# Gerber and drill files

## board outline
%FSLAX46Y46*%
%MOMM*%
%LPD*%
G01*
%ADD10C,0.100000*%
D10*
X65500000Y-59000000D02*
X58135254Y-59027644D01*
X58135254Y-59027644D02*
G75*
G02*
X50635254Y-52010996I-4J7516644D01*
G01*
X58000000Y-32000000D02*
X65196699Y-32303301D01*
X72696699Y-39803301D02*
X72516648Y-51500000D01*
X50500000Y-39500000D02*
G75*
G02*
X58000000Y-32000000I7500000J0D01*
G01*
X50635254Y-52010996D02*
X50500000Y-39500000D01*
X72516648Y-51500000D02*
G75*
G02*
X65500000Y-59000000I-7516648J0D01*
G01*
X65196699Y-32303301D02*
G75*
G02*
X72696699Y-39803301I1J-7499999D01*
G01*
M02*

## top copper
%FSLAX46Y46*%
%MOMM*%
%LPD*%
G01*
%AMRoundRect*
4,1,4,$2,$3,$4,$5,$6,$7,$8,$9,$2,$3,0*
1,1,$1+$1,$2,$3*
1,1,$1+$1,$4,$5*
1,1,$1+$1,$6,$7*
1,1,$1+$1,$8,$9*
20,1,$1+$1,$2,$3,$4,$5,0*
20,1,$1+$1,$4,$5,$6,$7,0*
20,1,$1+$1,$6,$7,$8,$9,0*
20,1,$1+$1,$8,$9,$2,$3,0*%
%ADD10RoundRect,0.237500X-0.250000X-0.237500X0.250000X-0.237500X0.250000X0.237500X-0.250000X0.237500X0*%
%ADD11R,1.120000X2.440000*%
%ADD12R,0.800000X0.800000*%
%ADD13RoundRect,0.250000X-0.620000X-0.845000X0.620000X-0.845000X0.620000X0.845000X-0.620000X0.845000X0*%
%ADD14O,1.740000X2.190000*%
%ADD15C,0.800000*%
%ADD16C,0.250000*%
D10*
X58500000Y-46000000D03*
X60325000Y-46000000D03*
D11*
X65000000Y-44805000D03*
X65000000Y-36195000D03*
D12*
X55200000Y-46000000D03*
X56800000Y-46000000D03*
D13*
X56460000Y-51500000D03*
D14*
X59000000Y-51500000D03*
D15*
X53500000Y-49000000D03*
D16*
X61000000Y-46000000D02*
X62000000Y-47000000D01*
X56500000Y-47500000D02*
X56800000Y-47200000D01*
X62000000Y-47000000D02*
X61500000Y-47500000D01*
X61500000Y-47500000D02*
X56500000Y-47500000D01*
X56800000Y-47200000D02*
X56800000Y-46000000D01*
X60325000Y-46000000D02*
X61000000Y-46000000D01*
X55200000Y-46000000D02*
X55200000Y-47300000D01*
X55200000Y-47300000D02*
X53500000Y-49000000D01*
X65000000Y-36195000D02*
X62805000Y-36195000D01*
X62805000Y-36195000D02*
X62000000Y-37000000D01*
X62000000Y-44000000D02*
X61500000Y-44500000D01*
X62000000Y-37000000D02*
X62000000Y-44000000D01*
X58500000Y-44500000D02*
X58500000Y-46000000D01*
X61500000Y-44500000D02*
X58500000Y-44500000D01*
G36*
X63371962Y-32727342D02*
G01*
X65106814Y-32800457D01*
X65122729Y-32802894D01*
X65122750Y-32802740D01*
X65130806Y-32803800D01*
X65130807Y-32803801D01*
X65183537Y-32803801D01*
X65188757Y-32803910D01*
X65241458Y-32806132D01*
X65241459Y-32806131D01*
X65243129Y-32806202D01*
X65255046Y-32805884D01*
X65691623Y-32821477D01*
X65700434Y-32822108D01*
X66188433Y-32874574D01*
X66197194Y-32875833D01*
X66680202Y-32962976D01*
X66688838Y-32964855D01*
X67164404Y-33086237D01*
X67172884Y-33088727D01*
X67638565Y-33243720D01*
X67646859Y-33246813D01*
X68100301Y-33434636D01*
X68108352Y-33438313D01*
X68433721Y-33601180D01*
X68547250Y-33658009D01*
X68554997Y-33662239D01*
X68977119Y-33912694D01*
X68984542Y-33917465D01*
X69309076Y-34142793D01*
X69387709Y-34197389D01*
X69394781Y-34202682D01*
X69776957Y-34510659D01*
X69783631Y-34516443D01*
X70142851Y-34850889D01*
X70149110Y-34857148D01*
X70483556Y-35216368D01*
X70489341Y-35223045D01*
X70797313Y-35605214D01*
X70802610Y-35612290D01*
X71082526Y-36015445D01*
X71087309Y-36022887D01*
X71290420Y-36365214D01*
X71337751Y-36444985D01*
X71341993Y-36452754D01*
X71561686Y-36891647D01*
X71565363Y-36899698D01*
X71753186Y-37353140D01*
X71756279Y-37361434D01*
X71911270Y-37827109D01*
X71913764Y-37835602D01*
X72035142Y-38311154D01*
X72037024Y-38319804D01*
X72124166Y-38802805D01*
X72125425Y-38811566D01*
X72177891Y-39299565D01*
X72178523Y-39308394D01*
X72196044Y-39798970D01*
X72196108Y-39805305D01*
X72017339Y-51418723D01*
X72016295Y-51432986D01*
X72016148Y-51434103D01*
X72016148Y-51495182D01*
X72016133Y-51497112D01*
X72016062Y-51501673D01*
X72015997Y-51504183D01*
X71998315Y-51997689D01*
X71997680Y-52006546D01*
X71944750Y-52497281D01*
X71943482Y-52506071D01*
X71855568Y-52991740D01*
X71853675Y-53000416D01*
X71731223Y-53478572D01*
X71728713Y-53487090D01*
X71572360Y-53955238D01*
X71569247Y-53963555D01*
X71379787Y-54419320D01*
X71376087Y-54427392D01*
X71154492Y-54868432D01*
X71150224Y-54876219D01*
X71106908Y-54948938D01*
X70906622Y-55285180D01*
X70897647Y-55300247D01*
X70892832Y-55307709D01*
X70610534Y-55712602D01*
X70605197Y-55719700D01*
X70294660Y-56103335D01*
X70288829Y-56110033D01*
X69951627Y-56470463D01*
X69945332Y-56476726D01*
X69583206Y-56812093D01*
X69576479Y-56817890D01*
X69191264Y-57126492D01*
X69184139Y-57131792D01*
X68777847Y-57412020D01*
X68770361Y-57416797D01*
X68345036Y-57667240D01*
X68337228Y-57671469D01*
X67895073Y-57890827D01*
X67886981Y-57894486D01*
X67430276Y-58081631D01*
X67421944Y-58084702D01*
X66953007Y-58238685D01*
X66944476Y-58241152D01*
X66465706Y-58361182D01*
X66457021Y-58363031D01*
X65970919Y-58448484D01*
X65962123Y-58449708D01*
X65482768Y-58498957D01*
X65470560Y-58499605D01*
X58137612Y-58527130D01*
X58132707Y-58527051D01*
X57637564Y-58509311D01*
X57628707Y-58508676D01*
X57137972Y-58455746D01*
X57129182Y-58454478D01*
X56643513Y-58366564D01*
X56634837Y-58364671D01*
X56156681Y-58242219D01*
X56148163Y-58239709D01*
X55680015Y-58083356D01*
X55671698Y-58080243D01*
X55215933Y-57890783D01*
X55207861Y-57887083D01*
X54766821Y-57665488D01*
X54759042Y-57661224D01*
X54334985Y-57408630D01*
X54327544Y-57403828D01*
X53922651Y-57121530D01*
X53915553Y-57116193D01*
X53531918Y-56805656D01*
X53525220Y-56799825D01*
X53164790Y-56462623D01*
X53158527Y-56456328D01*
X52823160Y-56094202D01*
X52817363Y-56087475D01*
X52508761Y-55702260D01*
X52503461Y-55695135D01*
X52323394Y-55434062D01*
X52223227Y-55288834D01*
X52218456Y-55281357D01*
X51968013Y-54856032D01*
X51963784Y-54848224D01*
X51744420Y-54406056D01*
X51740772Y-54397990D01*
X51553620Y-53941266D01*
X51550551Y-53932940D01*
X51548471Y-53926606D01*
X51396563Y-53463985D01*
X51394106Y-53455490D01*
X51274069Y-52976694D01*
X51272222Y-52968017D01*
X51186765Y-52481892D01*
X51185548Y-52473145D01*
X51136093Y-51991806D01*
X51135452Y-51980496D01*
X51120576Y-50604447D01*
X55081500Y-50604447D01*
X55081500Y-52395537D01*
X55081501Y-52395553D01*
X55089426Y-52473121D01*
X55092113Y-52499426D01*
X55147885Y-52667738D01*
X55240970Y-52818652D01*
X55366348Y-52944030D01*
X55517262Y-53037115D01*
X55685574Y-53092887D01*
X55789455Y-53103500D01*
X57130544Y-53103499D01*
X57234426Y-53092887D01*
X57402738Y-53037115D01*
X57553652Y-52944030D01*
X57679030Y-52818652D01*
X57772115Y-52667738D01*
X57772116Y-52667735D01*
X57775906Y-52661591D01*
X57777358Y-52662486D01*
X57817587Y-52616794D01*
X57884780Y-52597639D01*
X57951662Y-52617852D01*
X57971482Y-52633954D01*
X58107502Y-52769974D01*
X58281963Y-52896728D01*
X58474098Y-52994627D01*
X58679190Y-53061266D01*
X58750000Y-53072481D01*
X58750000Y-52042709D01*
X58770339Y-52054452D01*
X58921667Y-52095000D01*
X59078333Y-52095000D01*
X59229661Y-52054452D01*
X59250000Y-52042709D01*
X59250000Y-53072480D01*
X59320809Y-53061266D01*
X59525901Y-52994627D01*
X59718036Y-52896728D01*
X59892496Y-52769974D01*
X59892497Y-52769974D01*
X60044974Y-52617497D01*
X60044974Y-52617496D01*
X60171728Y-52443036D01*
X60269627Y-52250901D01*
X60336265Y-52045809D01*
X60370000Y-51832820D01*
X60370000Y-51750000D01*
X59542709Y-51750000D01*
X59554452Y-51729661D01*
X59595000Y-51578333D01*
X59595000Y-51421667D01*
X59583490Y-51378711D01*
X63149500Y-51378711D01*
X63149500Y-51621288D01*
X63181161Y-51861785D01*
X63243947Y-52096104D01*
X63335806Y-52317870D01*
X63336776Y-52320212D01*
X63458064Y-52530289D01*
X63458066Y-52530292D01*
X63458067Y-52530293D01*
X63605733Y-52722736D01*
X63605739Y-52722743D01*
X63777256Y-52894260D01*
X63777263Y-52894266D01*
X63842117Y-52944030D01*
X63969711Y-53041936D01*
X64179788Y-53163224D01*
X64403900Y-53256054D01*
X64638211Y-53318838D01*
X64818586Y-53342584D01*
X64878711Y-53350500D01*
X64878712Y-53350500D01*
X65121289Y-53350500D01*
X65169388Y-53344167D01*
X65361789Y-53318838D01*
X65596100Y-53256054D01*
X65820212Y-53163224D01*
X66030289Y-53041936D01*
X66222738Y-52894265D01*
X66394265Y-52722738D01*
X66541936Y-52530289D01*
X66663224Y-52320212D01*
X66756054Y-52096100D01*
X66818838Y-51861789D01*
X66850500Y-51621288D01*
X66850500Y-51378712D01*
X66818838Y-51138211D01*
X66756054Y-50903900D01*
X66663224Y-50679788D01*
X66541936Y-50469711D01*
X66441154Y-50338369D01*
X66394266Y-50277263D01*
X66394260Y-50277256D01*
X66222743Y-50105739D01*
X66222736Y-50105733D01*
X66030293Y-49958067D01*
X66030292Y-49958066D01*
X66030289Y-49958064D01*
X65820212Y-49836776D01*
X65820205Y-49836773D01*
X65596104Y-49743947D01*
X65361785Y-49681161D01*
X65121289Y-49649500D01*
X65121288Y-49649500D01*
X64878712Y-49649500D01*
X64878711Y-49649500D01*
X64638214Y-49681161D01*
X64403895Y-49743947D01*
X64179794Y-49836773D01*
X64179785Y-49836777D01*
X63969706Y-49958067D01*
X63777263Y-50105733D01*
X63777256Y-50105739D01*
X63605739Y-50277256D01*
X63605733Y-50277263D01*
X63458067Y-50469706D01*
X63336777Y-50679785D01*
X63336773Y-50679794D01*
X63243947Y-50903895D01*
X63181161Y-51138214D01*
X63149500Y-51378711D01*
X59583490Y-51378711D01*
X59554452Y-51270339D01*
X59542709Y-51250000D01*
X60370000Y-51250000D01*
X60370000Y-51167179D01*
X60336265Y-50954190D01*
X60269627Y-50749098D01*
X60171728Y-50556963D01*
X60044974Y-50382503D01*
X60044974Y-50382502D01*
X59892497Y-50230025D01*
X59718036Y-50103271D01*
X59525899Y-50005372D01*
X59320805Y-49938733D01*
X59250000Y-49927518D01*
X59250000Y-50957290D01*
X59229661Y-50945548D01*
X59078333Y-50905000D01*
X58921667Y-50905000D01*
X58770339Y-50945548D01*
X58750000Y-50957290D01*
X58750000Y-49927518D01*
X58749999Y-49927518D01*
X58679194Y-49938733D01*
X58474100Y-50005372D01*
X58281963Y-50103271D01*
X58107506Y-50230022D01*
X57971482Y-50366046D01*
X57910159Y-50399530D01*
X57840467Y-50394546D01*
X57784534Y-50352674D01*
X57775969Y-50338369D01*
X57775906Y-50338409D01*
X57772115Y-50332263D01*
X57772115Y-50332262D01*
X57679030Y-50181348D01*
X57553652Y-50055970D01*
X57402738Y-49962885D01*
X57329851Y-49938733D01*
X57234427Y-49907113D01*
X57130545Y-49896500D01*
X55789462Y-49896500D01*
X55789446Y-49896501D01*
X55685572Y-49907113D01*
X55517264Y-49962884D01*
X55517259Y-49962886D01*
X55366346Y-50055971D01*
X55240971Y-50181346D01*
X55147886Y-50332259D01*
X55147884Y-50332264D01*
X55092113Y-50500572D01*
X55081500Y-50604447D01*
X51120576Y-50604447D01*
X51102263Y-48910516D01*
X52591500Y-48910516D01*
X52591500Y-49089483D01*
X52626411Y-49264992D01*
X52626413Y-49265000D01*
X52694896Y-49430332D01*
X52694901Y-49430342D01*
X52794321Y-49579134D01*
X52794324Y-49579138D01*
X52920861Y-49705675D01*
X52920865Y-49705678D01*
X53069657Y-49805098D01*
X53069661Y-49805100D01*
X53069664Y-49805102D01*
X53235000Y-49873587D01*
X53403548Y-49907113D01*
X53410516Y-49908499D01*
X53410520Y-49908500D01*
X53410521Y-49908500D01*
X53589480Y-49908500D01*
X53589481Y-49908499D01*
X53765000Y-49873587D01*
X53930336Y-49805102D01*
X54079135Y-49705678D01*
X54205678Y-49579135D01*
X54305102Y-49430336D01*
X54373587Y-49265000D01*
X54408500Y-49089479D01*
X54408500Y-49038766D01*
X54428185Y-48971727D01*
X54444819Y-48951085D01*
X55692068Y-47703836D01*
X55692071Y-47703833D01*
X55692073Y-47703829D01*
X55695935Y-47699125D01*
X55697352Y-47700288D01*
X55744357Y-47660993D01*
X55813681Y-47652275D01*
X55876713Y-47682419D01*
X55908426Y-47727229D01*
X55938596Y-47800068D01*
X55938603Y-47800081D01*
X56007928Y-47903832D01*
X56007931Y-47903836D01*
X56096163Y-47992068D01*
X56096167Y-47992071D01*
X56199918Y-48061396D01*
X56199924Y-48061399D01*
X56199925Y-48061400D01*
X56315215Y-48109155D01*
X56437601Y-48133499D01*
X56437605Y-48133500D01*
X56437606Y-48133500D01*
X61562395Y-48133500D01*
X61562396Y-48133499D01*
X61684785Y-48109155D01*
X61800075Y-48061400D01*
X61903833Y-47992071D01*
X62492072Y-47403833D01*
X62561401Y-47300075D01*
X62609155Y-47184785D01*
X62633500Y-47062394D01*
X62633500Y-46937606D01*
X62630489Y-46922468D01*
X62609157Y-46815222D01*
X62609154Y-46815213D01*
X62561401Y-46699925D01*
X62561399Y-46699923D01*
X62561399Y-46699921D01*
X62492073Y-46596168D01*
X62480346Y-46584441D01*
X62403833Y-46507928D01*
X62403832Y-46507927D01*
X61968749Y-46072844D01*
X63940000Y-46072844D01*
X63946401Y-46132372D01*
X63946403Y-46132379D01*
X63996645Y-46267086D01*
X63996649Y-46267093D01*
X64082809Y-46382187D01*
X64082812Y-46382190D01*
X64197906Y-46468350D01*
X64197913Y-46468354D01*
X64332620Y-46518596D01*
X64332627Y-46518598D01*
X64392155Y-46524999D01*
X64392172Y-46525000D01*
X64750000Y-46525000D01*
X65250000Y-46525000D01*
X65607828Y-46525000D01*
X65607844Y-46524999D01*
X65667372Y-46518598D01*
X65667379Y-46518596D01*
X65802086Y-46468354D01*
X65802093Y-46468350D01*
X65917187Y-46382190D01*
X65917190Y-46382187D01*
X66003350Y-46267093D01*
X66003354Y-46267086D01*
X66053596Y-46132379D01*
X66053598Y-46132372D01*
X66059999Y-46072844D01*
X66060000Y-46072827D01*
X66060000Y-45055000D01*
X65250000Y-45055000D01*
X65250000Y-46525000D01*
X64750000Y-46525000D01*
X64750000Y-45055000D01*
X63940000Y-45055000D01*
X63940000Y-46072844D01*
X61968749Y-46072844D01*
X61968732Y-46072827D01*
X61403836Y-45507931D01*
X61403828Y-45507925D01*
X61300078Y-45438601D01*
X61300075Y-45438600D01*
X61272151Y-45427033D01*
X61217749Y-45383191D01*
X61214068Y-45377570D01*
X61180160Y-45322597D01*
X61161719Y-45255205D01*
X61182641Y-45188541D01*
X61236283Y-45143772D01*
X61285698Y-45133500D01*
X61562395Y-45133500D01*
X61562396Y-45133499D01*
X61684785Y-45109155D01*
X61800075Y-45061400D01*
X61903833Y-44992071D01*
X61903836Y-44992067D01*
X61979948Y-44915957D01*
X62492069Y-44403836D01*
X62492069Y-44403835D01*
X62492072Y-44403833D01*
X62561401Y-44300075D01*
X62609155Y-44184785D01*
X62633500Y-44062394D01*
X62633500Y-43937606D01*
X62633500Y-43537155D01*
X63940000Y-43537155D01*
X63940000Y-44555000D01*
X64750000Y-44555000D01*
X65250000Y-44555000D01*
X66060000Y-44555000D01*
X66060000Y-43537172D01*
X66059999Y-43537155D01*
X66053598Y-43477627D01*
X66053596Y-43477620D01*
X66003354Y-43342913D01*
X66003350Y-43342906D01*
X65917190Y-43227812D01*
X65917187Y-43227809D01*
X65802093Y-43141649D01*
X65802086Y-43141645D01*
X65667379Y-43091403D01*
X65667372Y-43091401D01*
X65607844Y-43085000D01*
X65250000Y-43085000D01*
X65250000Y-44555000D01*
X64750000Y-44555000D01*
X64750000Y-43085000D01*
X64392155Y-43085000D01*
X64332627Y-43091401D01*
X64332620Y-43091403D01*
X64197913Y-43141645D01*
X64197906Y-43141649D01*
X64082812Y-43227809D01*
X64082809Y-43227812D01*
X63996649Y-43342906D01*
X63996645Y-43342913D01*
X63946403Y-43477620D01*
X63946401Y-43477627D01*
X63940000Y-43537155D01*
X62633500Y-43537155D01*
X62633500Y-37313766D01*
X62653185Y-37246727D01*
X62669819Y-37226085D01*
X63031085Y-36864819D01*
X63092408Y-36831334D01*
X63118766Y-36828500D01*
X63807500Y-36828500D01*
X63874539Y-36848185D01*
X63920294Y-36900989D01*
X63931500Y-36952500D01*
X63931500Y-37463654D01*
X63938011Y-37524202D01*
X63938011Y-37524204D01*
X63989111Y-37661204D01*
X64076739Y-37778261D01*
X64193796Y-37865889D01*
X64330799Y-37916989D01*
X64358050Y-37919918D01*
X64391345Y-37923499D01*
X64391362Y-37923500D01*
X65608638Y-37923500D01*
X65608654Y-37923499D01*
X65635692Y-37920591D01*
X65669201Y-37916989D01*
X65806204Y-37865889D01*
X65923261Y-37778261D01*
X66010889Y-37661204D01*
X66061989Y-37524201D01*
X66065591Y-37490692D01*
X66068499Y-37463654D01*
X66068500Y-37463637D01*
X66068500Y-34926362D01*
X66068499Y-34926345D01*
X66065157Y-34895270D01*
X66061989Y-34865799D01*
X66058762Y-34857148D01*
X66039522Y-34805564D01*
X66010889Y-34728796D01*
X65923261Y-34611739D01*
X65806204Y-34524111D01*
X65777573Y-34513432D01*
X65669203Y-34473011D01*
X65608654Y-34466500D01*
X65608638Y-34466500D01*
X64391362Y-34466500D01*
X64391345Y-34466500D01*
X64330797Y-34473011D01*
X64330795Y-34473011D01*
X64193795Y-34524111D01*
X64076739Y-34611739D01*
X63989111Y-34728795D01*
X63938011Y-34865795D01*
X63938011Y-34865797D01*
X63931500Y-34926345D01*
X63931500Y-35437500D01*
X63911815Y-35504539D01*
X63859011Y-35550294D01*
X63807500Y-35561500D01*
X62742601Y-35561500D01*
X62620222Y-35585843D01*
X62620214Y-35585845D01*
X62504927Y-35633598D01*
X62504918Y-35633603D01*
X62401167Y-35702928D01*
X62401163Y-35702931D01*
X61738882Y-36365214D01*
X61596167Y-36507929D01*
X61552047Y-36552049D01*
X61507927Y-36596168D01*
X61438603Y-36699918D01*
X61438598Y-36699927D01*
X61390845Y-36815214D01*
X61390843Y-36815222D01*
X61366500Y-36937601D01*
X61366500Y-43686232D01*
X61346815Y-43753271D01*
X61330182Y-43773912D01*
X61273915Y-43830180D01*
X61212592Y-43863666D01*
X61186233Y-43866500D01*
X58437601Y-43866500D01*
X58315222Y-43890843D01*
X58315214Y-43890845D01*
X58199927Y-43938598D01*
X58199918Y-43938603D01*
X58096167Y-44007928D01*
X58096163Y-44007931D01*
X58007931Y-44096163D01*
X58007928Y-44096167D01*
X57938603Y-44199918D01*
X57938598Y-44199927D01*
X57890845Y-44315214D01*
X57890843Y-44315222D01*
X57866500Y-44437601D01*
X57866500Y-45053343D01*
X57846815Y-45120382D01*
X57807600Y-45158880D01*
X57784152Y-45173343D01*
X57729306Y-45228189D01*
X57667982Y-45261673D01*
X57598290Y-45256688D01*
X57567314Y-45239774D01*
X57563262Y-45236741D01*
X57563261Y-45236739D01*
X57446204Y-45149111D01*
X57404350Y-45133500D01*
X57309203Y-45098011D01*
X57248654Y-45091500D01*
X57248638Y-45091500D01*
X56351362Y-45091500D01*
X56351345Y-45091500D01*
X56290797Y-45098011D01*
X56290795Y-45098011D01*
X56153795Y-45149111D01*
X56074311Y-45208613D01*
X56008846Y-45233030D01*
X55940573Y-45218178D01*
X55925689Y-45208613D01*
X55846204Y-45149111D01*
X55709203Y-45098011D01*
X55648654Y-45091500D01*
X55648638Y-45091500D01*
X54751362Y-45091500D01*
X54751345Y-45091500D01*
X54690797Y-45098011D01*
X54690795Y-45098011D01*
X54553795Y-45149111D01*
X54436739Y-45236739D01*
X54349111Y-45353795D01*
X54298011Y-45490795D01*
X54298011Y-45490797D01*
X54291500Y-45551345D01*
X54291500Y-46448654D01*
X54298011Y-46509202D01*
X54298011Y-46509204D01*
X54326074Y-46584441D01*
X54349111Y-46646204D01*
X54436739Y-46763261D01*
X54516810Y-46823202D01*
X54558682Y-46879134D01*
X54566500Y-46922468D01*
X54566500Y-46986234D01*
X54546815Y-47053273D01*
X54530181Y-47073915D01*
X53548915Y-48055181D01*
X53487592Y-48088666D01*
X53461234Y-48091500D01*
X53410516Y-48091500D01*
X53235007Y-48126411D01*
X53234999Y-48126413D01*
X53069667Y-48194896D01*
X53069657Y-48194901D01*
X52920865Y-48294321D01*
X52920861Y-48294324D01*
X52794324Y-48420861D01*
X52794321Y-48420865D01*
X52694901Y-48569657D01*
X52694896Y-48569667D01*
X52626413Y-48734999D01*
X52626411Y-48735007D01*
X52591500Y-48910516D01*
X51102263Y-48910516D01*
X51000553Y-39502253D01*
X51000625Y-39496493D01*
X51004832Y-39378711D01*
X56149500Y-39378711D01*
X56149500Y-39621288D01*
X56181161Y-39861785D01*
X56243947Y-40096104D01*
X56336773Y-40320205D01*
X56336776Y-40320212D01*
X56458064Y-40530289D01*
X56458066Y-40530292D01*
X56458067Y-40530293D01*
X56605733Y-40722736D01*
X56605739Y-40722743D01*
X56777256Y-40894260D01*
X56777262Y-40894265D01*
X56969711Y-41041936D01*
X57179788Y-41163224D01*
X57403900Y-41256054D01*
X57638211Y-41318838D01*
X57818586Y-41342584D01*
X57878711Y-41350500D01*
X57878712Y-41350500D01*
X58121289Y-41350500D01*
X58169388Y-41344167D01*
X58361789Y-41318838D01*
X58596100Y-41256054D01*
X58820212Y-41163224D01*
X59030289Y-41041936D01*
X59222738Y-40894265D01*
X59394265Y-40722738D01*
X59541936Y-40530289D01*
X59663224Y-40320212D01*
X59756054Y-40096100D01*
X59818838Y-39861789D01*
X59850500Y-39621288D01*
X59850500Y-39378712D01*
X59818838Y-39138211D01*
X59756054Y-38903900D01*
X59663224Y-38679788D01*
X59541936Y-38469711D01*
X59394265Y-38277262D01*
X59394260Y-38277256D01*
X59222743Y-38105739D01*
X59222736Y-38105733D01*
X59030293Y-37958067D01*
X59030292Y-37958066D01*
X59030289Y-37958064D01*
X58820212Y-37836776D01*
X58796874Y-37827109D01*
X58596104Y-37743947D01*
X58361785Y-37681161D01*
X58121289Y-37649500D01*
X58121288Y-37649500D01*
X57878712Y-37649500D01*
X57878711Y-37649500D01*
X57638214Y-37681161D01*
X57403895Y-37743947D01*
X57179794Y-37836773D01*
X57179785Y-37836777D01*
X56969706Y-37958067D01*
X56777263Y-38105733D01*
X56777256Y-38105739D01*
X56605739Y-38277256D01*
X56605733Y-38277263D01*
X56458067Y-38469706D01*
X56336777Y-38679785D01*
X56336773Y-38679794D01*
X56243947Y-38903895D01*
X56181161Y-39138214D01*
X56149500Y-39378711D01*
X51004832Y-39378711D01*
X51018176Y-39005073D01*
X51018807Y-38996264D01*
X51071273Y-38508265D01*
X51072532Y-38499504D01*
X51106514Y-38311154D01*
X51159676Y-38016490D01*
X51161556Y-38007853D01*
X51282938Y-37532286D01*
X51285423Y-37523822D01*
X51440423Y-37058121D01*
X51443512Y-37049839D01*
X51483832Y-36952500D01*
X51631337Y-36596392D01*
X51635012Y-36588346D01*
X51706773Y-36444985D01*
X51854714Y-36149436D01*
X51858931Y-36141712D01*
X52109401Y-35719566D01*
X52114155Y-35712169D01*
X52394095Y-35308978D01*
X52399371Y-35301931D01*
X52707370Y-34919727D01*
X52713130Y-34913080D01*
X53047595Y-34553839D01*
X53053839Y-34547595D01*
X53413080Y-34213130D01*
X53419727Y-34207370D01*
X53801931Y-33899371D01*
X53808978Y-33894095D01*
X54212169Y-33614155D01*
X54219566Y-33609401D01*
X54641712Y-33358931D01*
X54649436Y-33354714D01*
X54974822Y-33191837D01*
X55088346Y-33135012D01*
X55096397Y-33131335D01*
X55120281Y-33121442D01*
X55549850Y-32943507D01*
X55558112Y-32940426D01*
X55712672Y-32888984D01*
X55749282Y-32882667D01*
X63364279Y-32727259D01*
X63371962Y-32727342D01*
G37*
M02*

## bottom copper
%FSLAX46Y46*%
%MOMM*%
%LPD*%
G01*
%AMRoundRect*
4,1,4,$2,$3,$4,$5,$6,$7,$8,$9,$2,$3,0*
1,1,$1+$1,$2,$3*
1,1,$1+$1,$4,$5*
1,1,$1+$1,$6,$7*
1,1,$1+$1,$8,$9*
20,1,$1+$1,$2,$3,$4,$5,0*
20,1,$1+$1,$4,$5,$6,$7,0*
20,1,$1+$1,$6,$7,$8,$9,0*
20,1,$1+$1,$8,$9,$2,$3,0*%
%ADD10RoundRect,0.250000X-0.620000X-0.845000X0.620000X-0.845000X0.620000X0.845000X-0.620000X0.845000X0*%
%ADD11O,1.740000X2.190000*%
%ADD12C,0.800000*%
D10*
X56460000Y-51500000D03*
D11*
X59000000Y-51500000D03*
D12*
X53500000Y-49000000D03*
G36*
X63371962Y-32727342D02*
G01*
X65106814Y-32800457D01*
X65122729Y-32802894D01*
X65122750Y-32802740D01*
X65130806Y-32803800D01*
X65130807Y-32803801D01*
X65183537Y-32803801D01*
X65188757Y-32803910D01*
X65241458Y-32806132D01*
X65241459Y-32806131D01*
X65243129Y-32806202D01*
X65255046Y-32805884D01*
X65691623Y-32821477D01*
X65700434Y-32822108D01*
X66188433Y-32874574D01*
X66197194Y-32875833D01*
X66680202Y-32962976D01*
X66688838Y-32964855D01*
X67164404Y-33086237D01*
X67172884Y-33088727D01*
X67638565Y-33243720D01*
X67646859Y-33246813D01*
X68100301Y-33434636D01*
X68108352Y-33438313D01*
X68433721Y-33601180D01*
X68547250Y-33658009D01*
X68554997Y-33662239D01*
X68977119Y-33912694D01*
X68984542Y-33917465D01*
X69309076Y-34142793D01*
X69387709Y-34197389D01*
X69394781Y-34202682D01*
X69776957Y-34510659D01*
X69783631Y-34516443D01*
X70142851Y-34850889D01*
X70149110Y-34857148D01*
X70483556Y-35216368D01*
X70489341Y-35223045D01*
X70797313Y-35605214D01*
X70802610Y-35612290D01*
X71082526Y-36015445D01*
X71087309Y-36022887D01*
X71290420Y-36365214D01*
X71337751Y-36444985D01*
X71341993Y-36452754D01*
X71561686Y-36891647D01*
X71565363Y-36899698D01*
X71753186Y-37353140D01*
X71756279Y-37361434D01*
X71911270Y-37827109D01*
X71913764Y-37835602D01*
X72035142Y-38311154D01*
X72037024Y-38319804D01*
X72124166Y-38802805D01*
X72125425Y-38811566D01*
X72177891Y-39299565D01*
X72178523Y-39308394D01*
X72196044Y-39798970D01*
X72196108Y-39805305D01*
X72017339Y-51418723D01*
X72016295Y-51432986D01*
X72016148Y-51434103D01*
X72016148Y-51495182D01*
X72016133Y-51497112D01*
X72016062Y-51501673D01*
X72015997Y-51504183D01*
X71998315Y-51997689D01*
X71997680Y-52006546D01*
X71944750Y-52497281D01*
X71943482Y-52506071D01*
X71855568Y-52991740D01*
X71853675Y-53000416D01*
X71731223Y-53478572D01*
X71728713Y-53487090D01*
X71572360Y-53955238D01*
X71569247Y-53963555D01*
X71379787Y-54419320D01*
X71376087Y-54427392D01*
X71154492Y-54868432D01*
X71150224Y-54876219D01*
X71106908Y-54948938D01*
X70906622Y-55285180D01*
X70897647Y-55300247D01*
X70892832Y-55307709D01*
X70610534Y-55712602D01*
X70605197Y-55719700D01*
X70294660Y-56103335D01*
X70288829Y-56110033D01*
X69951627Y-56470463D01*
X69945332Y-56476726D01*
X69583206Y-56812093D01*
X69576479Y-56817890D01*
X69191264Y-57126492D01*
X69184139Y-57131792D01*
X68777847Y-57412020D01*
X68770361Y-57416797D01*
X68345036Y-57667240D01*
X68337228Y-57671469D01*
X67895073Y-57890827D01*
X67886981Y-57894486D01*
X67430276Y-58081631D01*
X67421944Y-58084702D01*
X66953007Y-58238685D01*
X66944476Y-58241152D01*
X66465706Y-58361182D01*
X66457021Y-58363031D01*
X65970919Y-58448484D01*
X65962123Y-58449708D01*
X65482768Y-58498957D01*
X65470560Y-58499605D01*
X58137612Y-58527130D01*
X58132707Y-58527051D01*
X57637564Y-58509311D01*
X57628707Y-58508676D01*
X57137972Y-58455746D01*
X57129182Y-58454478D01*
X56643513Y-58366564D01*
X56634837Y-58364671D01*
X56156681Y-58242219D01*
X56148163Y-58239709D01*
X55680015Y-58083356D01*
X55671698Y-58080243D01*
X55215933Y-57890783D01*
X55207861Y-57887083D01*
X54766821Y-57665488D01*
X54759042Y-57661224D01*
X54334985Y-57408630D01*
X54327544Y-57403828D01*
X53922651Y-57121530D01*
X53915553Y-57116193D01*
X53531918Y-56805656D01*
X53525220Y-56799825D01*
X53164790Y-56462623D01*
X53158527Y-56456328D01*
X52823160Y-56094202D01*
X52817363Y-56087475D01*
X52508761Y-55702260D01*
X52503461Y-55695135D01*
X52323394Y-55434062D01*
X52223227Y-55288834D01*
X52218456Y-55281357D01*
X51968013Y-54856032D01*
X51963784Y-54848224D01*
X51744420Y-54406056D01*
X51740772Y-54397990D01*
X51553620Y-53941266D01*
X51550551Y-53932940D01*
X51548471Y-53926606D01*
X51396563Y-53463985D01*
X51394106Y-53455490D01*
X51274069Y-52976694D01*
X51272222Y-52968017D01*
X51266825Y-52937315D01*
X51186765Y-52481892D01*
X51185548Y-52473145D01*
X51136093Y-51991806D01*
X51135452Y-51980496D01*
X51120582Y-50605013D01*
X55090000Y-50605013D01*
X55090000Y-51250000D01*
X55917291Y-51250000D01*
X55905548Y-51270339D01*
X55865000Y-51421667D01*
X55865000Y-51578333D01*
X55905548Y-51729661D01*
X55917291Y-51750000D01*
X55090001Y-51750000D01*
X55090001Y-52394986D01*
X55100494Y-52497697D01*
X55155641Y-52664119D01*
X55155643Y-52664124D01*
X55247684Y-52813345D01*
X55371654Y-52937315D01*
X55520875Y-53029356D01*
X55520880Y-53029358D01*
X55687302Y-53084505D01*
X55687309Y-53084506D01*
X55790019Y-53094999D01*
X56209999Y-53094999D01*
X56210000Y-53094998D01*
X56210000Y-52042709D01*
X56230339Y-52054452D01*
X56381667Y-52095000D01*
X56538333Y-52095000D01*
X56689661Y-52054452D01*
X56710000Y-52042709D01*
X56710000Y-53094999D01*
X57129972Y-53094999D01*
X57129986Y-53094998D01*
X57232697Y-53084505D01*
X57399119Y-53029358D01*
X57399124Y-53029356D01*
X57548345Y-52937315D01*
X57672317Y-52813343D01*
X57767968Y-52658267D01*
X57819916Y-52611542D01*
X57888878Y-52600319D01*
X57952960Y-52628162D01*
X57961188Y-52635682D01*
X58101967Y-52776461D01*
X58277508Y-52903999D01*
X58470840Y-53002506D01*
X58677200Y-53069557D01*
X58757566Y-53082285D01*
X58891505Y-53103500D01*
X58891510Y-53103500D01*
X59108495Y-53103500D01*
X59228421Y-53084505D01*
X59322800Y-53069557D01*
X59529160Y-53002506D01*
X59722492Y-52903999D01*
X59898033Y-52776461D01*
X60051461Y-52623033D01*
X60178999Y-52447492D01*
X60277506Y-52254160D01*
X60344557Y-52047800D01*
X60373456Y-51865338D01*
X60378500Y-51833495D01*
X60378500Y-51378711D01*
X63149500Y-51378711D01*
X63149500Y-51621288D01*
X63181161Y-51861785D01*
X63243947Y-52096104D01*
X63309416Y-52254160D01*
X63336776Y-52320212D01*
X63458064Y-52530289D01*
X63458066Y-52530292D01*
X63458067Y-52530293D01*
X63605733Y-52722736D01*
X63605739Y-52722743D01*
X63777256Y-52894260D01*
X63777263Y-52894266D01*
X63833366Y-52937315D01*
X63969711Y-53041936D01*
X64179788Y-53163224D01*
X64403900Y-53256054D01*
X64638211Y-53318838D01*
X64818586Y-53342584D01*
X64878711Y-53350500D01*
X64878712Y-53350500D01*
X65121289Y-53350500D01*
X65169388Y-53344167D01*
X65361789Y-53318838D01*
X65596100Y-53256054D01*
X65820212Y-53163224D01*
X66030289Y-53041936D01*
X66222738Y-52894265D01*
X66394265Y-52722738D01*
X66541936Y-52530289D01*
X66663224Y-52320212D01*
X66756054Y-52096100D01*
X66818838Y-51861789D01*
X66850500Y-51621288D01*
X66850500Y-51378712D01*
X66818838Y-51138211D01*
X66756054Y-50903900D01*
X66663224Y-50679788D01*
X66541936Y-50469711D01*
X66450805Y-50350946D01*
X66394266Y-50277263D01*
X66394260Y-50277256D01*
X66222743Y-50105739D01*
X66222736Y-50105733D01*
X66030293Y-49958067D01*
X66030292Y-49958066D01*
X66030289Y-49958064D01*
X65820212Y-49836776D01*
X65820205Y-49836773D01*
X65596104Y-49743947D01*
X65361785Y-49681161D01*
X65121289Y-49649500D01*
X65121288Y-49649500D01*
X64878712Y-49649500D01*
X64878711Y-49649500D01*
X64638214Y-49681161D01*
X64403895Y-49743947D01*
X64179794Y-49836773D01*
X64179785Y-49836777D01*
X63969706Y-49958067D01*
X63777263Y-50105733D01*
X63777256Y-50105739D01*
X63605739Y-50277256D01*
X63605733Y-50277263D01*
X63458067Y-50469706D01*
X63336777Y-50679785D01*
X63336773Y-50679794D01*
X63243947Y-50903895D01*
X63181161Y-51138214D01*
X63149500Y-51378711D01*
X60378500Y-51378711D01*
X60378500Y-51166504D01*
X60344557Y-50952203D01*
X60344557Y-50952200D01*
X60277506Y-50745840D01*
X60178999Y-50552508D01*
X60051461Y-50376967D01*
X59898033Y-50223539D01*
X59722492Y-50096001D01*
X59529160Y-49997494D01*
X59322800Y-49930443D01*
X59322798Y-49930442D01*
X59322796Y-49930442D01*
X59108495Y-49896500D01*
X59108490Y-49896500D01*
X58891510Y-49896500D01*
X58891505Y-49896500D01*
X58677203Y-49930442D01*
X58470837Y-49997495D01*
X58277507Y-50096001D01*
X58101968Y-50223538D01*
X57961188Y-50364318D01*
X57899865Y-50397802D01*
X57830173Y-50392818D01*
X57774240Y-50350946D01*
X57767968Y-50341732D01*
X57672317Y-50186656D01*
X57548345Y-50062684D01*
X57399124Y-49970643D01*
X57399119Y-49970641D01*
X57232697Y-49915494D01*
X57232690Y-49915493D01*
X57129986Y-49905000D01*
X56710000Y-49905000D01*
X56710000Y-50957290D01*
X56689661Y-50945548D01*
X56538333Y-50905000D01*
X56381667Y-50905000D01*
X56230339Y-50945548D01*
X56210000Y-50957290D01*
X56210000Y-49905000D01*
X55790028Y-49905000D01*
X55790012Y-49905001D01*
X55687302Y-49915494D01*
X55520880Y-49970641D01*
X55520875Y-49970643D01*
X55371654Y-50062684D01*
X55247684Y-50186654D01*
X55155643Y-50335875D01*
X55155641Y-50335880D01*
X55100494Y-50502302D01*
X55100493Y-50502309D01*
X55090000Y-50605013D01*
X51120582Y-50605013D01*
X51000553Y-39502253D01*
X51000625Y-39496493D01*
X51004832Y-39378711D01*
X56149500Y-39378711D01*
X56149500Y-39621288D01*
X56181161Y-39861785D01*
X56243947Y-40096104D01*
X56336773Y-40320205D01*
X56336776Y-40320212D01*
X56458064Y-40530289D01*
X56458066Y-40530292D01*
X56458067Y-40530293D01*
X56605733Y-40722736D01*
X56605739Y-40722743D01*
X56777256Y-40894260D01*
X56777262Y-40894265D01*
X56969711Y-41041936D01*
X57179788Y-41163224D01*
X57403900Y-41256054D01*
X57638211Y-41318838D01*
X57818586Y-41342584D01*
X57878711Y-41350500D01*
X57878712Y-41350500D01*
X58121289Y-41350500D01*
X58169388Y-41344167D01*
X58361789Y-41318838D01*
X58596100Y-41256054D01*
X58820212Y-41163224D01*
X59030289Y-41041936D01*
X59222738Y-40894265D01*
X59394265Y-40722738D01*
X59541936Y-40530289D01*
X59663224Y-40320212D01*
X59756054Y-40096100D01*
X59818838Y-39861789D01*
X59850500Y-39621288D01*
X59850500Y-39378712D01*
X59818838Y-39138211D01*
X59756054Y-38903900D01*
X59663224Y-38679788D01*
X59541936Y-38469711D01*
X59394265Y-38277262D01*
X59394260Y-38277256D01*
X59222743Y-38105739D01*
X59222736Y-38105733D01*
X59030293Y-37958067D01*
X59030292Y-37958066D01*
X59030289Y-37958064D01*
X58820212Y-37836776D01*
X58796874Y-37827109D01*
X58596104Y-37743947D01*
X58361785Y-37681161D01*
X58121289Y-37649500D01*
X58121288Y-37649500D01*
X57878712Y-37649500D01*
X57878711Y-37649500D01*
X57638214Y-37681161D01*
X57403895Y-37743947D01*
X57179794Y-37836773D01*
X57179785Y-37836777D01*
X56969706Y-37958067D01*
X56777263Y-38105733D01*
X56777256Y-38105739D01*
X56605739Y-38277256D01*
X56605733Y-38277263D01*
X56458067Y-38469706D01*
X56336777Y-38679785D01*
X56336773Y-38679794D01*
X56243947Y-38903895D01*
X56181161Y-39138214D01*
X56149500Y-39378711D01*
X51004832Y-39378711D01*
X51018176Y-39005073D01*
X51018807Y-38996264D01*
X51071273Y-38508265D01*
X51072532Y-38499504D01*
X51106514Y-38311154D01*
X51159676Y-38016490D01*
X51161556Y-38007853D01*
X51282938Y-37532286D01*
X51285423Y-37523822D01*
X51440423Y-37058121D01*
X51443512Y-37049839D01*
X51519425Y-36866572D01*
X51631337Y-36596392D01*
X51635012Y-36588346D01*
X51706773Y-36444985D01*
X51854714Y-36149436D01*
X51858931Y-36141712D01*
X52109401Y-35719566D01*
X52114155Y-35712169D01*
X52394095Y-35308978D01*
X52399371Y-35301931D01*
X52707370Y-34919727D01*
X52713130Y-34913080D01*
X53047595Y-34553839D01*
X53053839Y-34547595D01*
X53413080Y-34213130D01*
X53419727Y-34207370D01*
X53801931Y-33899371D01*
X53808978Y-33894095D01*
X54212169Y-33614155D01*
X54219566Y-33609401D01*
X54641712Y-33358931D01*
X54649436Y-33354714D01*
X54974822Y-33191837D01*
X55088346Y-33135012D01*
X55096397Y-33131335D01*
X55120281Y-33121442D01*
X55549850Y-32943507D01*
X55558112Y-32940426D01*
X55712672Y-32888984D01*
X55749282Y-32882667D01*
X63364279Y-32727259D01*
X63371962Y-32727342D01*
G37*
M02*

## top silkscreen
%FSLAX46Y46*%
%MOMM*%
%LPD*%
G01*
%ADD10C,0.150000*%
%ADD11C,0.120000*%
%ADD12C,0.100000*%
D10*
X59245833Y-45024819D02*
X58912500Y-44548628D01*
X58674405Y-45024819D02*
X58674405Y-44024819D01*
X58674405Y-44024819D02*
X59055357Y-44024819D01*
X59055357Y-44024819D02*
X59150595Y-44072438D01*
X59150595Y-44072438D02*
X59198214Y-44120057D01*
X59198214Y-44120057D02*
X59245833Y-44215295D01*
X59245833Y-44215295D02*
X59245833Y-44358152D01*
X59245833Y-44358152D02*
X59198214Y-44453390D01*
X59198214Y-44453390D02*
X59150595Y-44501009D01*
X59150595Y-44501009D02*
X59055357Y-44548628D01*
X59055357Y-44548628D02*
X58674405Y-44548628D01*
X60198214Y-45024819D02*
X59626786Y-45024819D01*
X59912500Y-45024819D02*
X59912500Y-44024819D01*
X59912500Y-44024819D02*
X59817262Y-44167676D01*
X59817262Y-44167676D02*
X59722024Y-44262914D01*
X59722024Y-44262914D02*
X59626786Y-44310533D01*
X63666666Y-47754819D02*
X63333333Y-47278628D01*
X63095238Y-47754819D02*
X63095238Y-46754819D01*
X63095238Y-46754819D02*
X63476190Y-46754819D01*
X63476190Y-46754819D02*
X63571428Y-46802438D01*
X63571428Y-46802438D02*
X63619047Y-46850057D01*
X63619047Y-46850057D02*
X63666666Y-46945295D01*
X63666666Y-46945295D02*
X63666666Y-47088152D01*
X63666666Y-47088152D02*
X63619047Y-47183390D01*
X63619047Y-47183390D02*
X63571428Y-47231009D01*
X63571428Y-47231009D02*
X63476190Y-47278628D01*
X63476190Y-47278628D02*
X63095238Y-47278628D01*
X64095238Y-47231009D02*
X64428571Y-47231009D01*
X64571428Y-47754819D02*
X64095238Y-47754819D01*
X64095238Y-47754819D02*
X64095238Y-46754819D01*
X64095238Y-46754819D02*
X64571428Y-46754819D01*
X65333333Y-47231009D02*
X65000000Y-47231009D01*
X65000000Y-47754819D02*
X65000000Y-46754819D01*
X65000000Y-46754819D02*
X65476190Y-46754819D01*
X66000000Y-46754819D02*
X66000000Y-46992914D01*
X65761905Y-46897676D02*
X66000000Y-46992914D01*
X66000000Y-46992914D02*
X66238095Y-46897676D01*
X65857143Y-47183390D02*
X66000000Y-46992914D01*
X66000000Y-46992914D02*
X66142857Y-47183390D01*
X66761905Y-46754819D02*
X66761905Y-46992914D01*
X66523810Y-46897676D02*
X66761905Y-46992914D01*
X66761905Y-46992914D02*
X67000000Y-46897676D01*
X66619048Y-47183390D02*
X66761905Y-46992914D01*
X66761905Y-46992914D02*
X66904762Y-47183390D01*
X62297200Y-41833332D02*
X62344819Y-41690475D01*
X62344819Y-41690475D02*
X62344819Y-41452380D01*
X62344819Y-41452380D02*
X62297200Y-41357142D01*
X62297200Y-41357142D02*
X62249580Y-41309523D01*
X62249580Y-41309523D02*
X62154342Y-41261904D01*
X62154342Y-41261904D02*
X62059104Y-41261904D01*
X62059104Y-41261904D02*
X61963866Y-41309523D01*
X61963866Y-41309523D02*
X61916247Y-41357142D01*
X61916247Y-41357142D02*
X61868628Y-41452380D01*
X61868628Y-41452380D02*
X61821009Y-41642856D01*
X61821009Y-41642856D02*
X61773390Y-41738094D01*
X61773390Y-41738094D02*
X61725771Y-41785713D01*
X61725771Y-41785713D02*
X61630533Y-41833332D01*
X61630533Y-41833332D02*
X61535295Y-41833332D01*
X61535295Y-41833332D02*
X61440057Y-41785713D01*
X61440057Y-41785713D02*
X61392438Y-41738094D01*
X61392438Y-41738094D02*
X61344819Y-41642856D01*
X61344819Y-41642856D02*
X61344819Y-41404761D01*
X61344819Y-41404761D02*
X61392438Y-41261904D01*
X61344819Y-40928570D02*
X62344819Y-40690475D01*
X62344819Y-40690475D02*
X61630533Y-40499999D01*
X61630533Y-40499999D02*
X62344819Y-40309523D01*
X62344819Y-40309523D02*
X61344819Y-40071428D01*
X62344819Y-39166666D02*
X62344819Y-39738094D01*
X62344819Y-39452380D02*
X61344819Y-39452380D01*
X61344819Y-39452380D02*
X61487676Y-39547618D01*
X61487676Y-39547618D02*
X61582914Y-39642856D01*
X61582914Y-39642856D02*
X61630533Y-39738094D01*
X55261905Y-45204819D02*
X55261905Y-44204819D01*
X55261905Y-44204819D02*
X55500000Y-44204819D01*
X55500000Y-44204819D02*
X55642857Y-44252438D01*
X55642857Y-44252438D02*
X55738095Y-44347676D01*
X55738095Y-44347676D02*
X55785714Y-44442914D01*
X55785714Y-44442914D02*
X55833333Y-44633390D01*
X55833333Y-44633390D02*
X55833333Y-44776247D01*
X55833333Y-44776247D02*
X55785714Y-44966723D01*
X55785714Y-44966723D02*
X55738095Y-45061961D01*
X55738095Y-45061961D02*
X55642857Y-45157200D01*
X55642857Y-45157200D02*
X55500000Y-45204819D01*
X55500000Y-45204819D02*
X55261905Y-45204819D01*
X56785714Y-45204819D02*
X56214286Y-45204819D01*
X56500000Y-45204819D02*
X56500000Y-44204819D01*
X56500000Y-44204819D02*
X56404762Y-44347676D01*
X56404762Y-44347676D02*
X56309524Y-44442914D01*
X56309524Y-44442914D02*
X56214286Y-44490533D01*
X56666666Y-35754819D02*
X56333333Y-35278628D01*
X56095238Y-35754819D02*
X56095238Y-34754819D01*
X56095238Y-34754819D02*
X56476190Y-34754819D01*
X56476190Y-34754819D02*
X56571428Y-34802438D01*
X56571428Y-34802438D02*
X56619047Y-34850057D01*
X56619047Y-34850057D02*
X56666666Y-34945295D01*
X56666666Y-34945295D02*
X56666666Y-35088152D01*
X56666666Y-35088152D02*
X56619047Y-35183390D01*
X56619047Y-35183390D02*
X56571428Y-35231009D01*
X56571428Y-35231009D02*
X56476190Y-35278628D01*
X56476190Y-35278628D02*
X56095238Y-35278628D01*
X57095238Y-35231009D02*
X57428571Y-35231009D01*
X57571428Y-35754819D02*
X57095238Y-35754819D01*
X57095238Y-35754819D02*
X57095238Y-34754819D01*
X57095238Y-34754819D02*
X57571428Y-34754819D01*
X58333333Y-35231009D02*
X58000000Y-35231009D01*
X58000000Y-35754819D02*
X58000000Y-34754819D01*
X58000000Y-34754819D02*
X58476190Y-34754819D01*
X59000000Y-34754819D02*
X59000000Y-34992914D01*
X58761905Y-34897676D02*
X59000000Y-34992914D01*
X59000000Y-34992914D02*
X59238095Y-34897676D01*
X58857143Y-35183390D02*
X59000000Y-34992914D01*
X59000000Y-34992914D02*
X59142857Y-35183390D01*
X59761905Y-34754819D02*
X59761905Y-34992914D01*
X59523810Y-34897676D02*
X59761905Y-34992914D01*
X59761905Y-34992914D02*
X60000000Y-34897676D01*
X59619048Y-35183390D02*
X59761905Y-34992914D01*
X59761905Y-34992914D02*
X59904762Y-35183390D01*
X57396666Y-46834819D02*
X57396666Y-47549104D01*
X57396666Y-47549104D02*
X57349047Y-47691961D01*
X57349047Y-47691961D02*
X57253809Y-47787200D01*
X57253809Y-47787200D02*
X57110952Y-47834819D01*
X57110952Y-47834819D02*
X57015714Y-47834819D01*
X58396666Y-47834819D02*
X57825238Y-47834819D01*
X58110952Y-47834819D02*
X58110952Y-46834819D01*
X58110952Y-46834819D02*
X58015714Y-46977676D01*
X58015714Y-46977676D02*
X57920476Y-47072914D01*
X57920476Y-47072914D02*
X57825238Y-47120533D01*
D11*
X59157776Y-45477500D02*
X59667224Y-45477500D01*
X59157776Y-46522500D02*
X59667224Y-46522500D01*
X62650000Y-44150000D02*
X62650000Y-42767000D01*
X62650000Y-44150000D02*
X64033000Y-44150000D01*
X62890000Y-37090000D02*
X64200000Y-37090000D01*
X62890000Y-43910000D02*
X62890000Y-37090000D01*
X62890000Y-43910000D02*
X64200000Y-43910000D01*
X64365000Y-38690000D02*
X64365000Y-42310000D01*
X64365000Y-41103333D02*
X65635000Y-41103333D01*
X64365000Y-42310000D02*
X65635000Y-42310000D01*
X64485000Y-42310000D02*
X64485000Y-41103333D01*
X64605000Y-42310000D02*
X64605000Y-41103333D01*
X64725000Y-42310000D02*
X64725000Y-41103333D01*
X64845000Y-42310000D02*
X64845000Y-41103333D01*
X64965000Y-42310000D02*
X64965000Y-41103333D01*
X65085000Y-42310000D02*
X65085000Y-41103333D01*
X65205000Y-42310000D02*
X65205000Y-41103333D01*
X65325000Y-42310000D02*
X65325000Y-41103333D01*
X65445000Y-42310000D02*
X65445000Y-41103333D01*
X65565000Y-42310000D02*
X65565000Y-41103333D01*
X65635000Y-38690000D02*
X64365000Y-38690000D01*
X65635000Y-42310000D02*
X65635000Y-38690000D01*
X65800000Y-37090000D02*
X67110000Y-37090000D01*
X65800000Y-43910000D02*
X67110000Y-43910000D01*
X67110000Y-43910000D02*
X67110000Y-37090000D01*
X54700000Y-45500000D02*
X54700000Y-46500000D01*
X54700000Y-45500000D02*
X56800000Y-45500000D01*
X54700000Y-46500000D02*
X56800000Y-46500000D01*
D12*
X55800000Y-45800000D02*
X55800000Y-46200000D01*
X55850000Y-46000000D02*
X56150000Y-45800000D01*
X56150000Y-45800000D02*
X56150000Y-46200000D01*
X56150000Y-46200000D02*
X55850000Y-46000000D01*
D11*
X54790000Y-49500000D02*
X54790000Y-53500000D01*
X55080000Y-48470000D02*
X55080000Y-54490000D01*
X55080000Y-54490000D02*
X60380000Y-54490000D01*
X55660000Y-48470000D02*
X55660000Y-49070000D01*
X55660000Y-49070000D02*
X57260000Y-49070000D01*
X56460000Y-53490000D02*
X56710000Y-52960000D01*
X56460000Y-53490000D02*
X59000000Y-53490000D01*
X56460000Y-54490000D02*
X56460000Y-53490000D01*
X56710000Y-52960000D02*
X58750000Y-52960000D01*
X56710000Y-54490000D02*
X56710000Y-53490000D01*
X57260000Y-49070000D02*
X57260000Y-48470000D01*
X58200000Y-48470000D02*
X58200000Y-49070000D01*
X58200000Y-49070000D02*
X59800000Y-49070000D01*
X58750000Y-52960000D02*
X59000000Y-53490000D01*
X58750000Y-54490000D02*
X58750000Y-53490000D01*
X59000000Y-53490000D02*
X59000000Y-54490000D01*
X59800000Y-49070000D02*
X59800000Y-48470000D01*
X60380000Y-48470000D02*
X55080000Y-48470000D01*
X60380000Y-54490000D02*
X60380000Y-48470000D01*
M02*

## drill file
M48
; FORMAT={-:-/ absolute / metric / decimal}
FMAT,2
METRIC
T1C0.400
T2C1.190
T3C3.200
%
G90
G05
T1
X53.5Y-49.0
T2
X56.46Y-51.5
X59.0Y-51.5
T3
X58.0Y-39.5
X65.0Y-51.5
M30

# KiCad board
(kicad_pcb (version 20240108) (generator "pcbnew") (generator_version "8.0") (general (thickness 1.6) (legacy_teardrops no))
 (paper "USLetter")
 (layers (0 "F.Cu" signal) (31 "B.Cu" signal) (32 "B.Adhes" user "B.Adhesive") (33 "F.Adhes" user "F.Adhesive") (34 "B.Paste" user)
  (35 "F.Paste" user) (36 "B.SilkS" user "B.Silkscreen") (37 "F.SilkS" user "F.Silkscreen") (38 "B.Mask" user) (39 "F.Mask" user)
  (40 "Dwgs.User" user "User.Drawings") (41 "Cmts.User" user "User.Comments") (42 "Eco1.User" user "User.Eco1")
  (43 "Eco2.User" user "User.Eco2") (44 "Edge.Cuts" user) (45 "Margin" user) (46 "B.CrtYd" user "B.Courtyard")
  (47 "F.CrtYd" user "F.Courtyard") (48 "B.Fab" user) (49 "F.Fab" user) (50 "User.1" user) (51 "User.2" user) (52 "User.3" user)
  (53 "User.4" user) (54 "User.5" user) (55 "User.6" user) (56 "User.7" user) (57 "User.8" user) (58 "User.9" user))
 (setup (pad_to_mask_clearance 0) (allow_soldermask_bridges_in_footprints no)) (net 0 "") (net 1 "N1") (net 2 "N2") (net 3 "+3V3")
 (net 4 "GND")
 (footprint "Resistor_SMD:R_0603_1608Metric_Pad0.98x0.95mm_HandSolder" (layer "F.Cu") (at 59.4125 46)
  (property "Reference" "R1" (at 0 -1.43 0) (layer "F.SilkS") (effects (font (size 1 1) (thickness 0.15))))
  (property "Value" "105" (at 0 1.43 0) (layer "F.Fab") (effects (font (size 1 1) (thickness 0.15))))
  (fp_line (start -0.254724 -0.5225) (end 0.254724 -0.5225) (stroke (width 0.12) (type solid)) (layer "F.SilkS"))
  (fp_line (start -0.254724 0.5225) (end 0.254724 0.5225) (stroke (width 0.12) (type solid)) (layer "F.SilkS"))
  (pad "1" smd roundrect (at -0.9125 0) (size 0.975 0.95) (layers "F.Cu" "F.Paste" "F.Mask") (roundrect_rratio 0.25) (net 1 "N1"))
  (pad "2" smd roundrect (at 0.9125 0) (size 0.975 0.95) (layers "F.Cu" "F.Paste" "F.Mask") (roundrect_rratio 0.25) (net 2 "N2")))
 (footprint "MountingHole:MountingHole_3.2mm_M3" (layer "F.Cu") (at 65 51.5)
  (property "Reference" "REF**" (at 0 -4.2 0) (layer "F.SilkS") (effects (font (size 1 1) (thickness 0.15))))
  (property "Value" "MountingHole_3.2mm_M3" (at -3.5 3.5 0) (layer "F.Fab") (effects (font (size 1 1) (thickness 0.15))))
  (pad "" np_thru_hole circle (at 0 0) (size 3.2 3.2) (drill 3.2) (layers "*.Cu" "*.Mask")))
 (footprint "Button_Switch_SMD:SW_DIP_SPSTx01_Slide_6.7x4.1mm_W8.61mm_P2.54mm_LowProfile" (layer "F.Cu") (at 65 40.5 90)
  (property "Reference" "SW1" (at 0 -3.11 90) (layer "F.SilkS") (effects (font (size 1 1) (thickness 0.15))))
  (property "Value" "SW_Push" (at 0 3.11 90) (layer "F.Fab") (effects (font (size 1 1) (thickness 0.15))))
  (fp_line (start -3.65 -2.35) (end -2.267 -2.35) (stroke (width 0.12) (type solid)) (layer "F.SilkS"))
  (fp_line (start -3.65 -2.35) (end -3.65 -0.967) (stroke (width 0.12) (type solid)) (layer "F.SilkS"))
  (fp_line (start 3.41 -2.11) (end 3.41 -0.8) (stroke (width 0.12) (type solid)) (layer "F.SilkS"))
  (fp_line (start -3.41 -2.11) (end 3.41 -2.11) (stroke (width 0.12) (type solid)) (layer "F.SilkS"))
  (fp_line (start -3.41 -2.11) (end -3.41 -0.8) (stroke (width 0.12) (type solid)) (layer "F.SilkS"))
  (fp_line (start 1.81 -0.635) (end -1.81 -0.635) (stroke (width 0.12) (type solid)) (layer "F.SilkS"))
  (fp_line (start -0.603333 -0.635) (end -0.603333 0.635) (stroke (width 0.12) (type solid)) (layer "F.SilkS"))
  (fp_line (start -1.81 -0.635) (end -1.81 0.635) (stroke (width 0.12) (type solid)) (layer "F.SilkS"))
  (fp_line (start -1.81 -0.515) (end -0.603333 -0.515) (stroke (width 0.12) (type solid)) (layer "F.SilkS"))
  (fp_line (start -1.81 -0.395) (end -0.603333 -0.395) (stroke (width 0.12) (type solid)) (layer "F.SilkS"))
  (fp_line (start -1.81 -0.275) (end -0.603333 -0.275) (stroke (width 0.12) (type solid)) (layer "F.SilkS"))
  (fp_line (start -1.81 -0.155) (end -0.603333 -0.155) (stroke (width 0.12) (type solid)) (layer "F.SilkS"))
  (fp_line (start -1.81 -0.035) (end -0.603333 -0.035) (stroke (width 0.12) (type solid)) (layer "F.SilkS"))
  (fp_line (start -1.81 0.085) (end -0.603333 0.085) (stroke (width 0.12) (type solid)) (layer "F.SilkS"))
  (fp_line (start -1.81 0.205) (end -0.603333 0.205) (stroke (width 0.12) (type solid)) (layer "F.SilkS"))
  (fp_line (start -1.81 0.325) (end -0.603333 0.325) (stroke (width 0.12) (type solid)) (layer "F.SilkS"))
  (fp_line (start -1.81 0.445) (end -0.603333 0.445) (stroke (width 0.12) (type solid)) (layer "F.SilkS"))
  (fp_line (start -1.81 0.565) (end -0.603333 0.565) (stroke (width 0.12) (type solid)) (layer "F.SilkS"))
  (fp_line (start 1.81 0.635) (end 1.81 -0.635) (stroke (width 0.12) (type solid)) (layer "F.SilkS"))
  (fp_line (start -1.81 0.635) (end 1.81 0.635) (stroke (width 0.12) (type solid)) (layer "F.SilkS"))
  (fp_line (start 3.41 0.8) (end 3.41 2.11) (stroke (width 0.12) (type solid)) (layer "F.SilkS"))
  (fp_line (start -3.41 0.8) (end -3.41 2.11) (stroke (width 0.12) (type solid)) (layer "F.SilkS"))
  (fp_line (start -3.41 2.11) (end 3.41 2.11) (stroke (width 0.12) (type solid)) (layer "F.SilkS"))
  (pad "1" smd rect (at -4.305 0 90) (size 2.44 1.12) (layers "F.Cu" "F.Paste" "F.Mask") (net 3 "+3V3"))
  (pad "2" smd rect (at 4.305 0 90) (size 2.44 1.12) (layers "F.Cu" "F.Paste" "F.Mask") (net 1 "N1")))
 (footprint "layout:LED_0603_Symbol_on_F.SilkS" (layer "F.Cu") (at 56 46)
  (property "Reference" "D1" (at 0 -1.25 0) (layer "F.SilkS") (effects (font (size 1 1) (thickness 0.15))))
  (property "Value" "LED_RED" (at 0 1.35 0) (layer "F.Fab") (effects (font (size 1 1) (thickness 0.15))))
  (fp_line (start -1.3 -0.5) (end -1.3 0.5) (stroke (width 0.12) (type solid)) (layer "F.SilkS"))
  (fp_line (start -1.3 -0.5) (end 0.8 -0.5) (stroke (width 0.12) (type solid)) (layer "F.SilkS"))
  (fp_line (start -1.3 0.5) (end 0.8 0.5) (stroke (width 0.12) (type solid)) (layer "F.SilkS"))
  (fp_line (start -0.2 -0.2) (end -0.2 0.2) (stroke (width 0.1) (type solid)) (layer "F.SilkS"))
  (fp_line (start -0.15 0) (end 0.15 -0.2) (stroke (width 0.1) (type solid)) (layer "F.SilkS"))
  (fp_line (start 0.15 -0.2) (end 0.15 0.2) (stroke (width 0.1) (type solid)) (layer "F.SilkS"))
  (fp_line (start 0.15 0.2) (end -0.15 0) (stroke (width 0.1) (type solid)) (layer "F.SilkS"))
  (pad "1" smd rect (at -0.8 0 180) (size 0.8 0.8) (layers "F.Cu" "F.Paste" "F.Mask") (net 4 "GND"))
  (pad "2" smd rect (at 0.8 0 180) (size 0.8 0.8) (layers "F.Cu" "F.Paste" "F.Mask") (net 2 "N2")))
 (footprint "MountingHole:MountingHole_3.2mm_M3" (layer "F.Cu") (at 58 39.5)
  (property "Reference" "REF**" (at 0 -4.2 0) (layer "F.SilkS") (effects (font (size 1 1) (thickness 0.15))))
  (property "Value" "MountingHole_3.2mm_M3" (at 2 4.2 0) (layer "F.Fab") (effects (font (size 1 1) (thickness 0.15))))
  (pad "" np_thru_hole circle (at 0 0) (size 3.2 3.2) (drill 3.2) (layers "*.Cu" "*.Mask")))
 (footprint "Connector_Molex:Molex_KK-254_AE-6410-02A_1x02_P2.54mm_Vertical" (layer "F.Cu") (at 56.46 51.5)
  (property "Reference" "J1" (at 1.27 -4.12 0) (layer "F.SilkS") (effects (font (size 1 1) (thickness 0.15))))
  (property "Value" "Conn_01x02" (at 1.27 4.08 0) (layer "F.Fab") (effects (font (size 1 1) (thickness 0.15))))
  (fp_line (start -1.67 -2) (end -1.67 2) (stroke (width 0.12) (type solid)) (layer "F.SilkS"))
  (fp_line (start -1.38 -3.03) (end -1.38 2.99) (stroke (width 0.12) (type solid)) (layer "F.SilkS"))
  (fp_line (start -1.38 2.99) (end 3.92 2.99) (stroke (width 0.12) (type solid)) (layer "F.SilkS"))
  (fp_line (start -0.8 -3.03) (end -0.8 -2.43) (stroke (width 0.12) (type solid)) (layer "F.SilkS"))
  (fp_line (start -0.8 -2.43) (end 0.8 -2.43) (stroke (width 0.12) (type solid)) (layer "F.SilkS"))
  (fp_line (start 0 1.99) (end 0.25 1.46) (stroke (width 0.12) (type solid)) (layer "F.SilkS"))
  (fp_line (start 0 1.99) (end 2.54 1.99) (stroke (width 0.12) (type solid)) (layer "F.SilkS"))
  (fp_line (start 0 2.99) (end 0 1.99) (stroke (width 0.12) (type solid)) (layer "F.SilkS"))
  (fp_line (start 0.25 1.46) (end 2.29 1.46) (stroke (width 0.12) (type solid)) (layer "F.SilkS"))
  (fp_line (start 0.25 2.99) (end 0.25 1.99) (stroke (width 0.12) (type solid)) (layer "F.SilkS"))
  (fp_line (start 0.8 -2.43) (end 0.8 -3.03) (stroke (width 0.12) (type solid)) (layer "F.SilkS"))
  (fp_line (start 1.74 -3.03) (end 1.74 -2.43) (stroke (width 0.12) (type solid)) (layer "F.SilkS"))
  (fp_line (start 1.74 -2.43) (end 3.34 -2.43) (stroke (width 0.12) (type solid)) (layer "F.SilkS"))
  (fp_line (start 2.29 1.46) (end 2.54 1.99) (stroke (width 0.12) (type solid)) (layer "F.SilkS"))
  (fp_line (start 2.29 2.99) (end 2.29 1.99) (stroke (width 0.12) (type solid)) (layer "F.SilkS"))
  (fp_line (start 2.54 1.99) (end 2.54 2.99) (stroke (width 0.12) (type solid)) (layer "F.SilkS"))
  (fp_line (start 3.34 -2.43) (end 3.34 -3.03) (stroke (width 0.12) (type solid)) (layer "F.SilkS"))
  (fp_line (start 3.92 -3.03) (end -1.38 -3.03) (stroke (width 0.12) (type solid)) (layer "F.SilkS"))
  (fp_line (start 3.92 2.99) (end 3.92 -3.03) (stroke (width 0.12) (type solid)) (layer "F.SilkS"))
  (pad "1" thru_hole roundrect (at 0 0) (size 1.74 2.19) (drill 1.19) (layers "*.Cu" "*.Mask") (remove_unused_layers no)
   (roundrect_rratio 0.143678) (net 4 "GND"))
  (pad "2" thru_hole oval (at 2.54 0) (size 1.74 2.19) (drill 1.19) (layers "*.Cu" "*.Mask") (remove_unused_layers no) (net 3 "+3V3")))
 (gr_line (start 65.5 59) (end 58.135254 59.027644) (stroke (width 0.1) (type default)) (layer "Edge.Cuts"))
 (gr_arc (start 58.135254 59.027644) (mid 53 57) (end 50.635254 52.010996) (stroke (width 0.1) (type default)) (layer "Edge.Cuts"))
 (gr_line (start 58 32) (end 65.196699 32.303301) (stroke (width 0.1) (type default)) (layer "Edge.Cuts"))
 (gr_line (start 72.696699 39.803301) (end 72.516648 51.5) (stroke (width 0.1) (type default)) (layer "Edge.Cuts"))
 (gr_arc (start 50.5 39.5) (mid 52.696699 34.196699) (end 58 32) (stroke (width 0.1) (type default)) (layer "Edge.Cuts"))
 (gr_line (start 50.635254 52.010996) (end 50.5 39.5) (stroke (width 0.1) (type default)) (layer "Edge.Cuts"))
 (gr_arc (start 72.516648 51.5) (mid 70.489004 56.635254) (end 65.5 59) (stroke (width 0.1) (type default)) (layer "Edge.Cuts"))
 (gr_arc (start 65.196699 32.303301) (mid 70.5 34.5) (end 72.696699 39.803301) (stroke (width 0.1) (type default)) (layer "Edge.Cuts"))
 (segment (start 61 46) (end 62 47) (width 0.25) (layer "F.Cu") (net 2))
 (segment (start 56.5 47.5) (end 56.8 47.2) (width 0.25) (layer "F.Cu") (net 2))
 (segment (start 62 47) (end 61.5 47.5) (width 0.25) (layer "F.Cu") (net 2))
 (segment (start 61.5 47.5) (end 56.5 47.5) (width 0.25) (layer "F.Cu") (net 2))
 (segment (start 56.8 47.2) (end 56.8 46) (width 0.25) (layer "F.Cu") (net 2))
 (segment (start 60.325 46) (end 61 46) (width 0.25) (layer "F.Cu") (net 2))
 (segment (start 55.2 46) (end 55.2 47.3) (width 0.25) (layer "F.Cu") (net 4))
 (segment (start 55.2 47.3) (end 53.5 49) (width 0.25) (layer "F.Cu") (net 4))
 (via (at 53.5 49) (size 0.8) (drill 0.4) (layers "F.Cu" "B.Cu") (free yes) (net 4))
 (segment (start 65 36.195) (end 62.805 36.195) (width 0.25) (layer "F.Cu") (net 1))
 (segment (start 62.805 36.195) (end 62 37) (width 0.25) (layer "F.Cu") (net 1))
 (segment (start 62 44) (end 61.5 44.5) (width 0.25) (layer "F.Cu") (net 1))
 (segment (start 62 37) (end 62 44) (width 0.25) (layer "F.Cu") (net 1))
 (segment (start 58.5 44.5) (end 58.5 46) (width 0.25) (layer "F.Cu") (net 1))
 (segment (start 61.5 44.5) (end 58.5 44.5) (width 0.25) (layer "F.Cu") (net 1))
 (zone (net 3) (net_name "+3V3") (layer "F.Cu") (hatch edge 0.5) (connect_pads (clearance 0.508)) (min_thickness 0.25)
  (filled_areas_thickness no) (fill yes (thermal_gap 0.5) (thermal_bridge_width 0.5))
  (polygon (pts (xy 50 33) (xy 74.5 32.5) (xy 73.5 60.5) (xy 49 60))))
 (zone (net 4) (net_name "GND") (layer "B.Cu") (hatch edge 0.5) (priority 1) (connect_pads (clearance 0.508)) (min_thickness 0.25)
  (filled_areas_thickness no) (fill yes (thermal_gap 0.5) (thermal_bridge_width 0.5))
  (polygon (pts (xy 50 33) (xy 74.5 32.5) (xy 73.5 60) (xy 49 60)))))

